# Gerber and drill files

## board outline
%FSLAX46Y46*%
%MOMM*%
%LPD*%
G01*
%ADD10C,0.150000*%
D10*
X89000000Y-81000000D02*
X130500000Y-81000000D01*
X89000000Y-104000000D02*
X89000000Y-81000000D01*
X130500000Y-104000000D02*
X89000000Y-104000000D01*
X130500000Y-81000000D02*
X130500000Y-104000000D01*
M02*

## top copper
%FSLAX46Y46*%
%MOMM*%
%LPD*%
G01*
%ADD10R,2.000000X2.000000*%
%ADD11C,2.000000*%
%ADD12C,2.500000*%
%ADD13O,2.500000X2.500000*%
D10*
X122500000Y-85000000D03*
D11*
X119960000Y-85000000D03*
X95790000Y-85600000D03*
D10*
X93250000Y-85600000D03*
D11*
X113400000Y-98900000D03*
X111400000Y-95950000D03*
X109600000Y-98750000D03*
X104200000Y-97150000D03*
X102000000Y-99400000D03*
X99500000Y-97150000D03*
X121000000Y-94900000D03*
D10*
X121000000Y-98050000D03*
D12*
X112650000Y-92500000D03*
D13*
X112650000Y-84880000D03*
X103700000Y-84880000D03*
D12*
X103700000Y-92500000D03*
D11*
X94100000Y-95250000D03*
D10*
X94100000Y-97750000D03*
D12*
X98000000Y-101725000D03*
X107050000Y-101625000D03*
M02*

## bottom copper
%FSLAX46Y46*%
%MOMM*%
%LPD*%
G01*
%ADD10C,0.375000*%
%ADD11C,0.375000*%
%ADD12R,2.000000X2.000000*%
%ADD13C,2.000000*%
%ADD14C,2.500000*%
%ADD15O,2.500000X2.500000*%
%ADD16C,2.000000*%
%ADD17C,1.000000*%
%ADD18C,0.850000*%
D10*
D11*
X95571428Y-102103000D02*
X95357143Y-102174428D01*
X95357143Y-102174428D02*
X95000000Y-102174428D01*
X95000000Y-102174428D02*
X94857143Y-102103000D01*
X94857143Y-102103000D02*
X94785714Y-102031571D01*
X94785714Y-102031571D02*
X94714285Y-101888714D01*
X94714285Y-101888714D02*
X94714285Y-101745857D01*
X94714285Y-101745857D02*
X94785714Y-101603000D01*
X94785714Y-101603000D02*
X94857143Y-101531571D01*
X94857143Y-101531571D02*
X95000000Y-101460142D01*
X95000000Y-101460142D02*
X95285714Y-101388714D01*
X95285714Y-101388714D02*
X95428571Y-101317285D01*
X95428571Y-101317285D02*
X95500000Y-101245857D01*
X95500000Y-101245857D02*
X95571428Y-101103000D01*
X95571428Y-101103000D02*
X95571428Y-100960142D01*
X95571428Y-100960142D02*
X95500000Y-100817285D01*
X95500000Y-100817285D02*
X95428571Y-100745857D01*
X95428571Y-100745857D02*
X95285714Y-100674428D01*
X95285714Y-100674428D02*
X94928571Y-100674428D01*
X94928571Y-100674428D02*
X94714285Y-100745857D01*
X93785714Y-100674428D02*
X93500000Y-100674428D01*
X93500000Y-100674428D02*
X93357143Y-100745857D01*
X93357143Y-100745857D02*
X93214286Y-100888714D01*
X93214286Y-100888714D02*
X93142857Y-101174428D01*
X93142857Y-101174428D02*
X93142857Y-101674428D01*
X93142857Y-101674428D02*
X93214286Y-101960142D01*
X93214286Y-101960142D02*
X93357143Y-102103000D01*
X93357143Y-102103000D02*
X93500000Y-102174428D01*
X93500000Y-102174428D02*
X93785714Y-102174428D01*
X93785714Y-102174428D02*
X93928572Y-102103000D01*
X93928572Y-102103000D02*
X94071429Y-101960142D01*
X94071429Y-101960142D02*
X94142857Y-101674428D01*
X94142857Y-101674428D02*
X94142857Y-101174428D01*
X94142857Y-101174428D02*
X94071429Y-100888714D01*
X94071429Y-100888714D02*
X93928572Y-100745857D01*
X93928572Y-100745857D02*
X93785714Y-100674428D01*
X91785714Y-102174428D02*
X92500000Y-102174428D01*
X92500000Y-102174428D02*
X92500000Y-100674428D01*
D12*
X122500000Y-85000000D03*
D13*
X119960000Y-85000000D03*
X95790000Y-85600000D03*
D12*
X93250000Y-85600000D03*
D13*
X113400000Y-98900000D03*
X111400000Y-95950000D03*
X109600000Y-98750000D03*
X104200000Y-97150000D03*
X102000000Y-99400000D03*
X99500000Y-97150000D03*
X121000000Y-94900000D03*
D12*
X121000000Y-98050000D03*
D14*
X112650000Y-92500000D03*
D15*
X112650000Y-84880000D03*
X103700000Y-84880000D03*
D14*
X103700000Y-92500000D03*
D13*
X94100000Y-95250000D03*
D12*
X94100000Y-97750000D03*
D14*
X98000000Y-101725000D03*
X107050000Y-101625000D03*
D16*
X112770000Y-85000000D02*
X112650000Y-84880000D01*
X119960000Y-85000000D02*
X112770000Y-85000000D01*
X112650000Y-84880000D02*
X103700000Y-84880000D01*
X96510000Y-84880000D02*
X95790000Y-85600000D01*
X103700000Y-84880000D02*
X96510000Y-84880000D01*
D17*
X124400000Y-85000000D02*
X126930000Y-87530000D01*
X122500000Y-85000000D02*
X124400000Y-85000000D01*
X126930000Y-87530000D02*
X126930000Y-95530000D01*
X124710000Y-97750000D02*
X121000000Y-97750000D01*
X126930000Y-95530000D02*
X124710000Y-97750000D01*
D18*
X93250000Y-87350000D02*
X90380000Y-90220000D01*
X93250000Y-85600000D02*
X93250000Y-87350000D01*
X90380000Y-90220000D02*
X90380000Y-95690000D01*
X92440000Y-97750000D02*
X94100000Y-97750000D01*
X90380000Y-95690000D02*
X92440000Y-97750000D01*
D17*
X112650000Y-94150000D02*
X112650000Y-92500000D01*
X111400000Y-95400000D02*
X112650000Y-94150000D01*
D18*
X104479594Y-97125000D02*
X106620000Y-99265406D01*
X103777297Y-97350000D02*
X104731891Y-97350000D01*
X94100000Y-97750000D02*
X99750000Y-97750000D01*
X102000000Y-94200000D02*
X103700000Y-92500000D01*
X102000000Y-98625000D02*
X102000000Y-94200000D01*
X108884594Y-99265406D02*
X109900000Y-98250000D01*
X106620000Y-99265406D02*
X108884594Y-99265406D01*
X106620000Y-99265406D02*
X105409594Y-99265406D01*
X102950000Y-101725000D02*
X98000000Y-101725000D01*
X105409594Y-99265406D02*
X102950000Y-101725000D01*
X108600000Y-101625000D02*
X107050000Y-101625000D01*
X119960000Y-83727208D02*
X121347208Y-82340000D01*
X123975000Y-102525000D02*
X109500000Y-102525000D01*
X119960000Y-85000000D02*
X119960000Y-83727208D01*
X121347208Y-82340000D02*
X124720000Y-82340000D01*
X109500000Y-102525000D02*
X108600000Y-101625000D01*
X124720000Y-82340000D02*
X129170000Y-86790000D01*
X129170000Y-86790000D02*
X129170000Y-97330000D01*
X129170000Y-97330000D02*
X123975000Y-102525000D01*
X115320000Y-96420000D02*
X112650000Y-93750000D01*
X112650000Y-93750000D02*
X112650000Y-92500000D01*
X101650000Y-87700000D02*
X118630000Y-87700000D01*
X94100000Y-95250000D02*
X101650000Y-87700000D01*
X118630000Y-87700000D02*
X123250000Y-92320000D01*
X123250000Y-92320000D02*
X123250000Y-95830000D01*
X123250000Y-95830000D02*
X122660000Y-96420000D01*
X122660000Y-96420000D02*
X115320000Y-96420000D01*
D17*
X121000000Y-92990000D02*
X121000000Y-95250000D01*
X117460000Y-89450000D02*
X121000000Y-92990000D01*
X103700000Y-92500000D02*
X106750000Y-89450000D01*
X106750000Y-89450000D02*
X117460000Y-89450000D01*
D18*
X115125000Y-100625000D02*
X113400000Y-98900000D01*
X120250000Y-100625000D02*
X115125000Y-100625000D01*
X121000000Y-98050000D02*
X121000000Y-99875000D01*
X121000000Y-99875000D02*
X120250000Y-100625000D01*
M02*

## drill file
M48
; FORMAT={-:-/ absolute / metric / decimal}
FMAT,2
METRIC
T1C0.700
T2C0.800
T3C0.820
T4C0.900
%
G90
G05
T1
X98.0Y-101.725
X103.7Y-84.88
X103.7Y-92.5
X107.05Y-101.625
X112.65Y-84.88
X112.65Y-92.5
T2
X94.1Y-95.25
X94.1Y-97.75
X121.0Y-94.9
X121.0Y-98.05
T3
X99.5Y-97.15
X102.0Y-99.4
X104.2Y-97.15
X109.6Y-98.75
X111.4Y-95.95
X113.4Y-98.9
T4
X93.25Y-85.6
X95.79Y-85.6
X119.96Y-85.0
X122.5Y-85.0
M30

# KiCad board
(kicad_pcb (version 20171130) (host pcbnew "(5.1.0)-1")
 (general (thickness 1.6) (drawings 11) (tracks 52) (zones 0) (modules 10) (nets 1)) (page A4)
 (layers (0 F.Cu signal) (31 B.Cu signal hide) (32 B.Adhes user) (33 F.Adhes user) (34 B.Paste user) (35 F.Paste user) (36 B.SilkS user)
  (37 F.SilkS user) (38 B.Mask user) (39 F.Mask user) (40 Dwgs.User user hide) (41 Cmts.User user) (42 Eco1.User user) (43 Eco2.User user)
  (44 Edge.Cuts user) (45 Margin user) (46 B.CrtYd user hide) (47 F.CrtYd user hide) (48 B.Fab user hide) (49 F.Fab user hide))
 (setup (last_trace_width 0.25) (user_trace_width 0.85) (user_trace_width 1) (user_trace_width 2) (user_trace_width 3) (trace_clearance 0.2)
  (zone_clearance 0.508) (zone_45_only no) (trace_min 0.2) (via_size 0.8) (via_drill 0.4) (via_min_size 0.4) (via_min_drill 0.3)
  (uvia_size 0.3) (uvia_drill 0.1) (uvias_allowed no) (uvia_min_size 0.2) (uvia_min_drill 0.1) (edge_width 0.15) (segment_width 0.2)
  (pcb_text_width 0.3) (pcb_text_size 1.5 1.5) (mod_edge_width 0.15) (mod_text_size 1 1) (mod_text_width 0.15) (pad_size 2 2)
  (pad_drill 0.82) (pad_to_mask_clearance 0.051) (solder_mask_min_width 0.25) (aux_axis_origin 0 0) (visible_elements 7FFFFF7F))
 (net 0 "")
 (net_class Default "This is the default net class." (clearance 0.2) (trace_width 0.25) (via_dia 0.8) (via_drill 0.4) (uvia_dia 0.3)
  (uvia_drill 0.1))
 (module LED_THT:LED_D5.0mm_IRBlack (layer F.Cu) (at 122.5 85 180)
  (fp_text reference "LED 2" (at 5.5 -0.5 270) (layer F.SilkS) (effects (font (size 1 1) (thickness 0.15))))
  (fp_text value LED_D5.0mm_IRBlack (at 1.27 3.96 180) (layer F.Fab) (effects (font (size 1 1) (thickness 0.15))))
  (pad 1 thru_hole rect (at 0 0 180) (size 2 2) (drill 0.9) (layers *.Cu *.Mask))
  (pad 2 thru_hole circle (at 2.54 0 180) (size 2 2) (drill 0.9) (layers *.Cu *.Mask)))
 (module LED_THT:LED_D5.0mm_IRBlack (layer F.Cu) (at 93.25 85.6)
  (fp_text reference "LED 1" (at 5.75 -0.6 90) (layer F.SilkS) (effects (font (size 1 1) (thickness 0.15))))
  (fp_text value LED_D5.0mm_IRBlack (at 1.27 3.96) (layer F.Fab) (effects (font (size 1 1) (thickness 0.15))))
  (pad 2 thru_hole circle (at 2.54 0) (size 2 2) (drill 0.9) (layers *.Cu *.Mask))
  (pad 1 thru_hole rect (at 0 0) (size 2 2) (drill 0.9) (layers *.Cu *.Mask)))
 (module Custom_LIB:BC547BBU (layer F.Cu) (at 111.4 97.85)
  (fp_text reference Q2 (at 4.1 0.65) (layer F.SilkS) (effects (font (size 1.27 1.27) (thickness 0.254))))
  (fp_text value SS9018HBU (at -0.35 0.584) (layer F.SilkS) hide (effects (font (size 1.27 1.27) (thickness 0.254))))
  (pad 3 thru_hole circle (at 2 1.05) (size 2 2) (drill 0.82) (layers *.Cu *.Mask))
  (pad 2 thru_hole circle (at 0 -1.9) (size 2 2) (drill 0.82) (layers *.Cu *.Mask))
  (pad 1 thru_hole circle (at -1.8 0.9) (size 2 2) (drill 0.82) (layers *.Cu *.Mask)))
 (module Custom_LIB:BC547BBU (layer F.Cu) (at 102 97.5 180)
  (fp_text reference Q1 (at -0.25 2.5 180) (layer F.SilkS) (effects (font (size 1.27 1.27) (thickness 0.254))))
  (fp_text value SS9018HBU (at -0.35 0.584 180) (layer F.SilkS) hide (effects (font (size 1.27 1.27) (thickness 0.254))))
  (pad 1 thru_hole circle (at -2.2 0.35 180) (size 2 2) (drill 0.82) (layers *.Cu *.Mask))
  (pad 2 thru_hole circle (at 0 -1.9 180) (size 2 2) (drill 0.82) (layers *.Cu *.Mask))
  (pad 3 thru_hole circle (at 2.5 0.35 180) (size 2 2) (drill 0.82) (layers *.Cu *.Mask)))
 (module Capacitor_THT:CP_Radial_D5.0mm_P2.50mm (layer F.Cu) (at 121 97.75 90)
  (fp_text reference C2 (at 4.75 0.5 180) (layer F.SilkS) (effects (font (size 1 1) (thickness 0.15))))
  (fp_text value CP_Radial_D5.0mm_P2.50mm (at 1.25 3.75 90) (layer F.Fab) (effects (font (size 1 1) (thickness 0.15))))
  (pad 2 thru_hole circle (at 2.85 0 90) (size 2 2) (drill 0.8) (layers *.Cu *.Mask))
  (pad 1 thru_hole rect (at -0.3 0 90) (size 2 2) (drill 0.8) (layers *.Cu *.Mask)))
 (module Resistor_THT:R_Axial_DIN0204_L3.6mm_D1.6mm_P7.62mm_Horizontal (layer F.Cu) (at 112.65 92.5 90)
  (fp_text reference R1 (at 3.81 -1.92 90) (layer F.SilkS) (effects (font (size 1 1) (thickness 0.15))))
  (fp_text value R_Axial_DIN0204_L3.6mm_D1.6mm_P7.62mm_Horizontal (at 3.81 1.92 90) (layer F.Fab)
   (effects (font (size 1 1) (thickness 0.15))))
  (pad 1 thru_hole circle (at 0 0 90) (size 2.5 2.5) (drill 0.7) (layers *.Cu *.Mask))
  (pad 2 thru_hole oval (at 7.62 0 90) (size 2.5 2.5) (drill 0.7) (layers *.Cu *.Mask)))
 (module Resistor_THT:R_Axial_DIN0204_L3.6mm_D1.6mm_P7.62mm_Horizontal (layer F.Cu) (at 103.7 92.5 90)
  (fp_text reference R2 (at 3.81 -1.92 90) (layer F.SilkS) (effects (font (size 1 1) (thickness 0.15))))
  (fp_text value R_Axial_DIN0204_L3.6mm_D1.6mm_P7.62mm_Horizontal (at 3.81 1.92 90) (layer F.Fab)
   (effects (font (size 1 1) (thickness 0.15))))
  (pad 2 thru_hole oval (at 7.62 0 90) (size 2.5 2.5) (drill 0.7) (layers *.Cu *.Mask))
  (pad 1 thru_hole circle (at 0 0 90) (size 2.5 2.5) (drill 0.7) (layers *.Cu *.Mask)))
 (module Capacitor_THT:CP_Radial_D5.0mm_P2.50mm (layer F.Cu) (at 94.1 97.75 90)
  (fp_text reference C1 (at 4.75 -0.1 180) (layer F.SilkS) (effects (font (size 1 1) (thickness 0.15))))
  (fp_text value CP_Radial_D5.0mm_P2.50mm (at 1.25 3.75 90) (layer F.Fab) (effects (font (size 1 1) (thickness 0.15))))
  (pad 2 thru_hole circle (at 2.5 0 90) (size 2 2) (drill 0.8) (layers *.Cu *.Mask))
  (pad 1 thru_hole rect (at 0 0 90) (size 2 2) (drill 0.8) (layers *.Cu *.Mask)))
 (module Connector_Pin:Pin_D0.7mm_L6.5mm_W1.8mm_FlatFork (layer F.Cu) (at 98 101.725)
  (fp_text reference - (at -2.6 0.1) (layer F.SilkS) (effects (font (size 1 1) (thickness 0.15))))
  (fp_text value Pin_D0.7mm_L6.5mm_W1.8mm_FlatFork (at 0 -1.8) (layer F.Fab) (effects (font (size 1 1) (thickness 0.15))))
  (pad 1 thru_hole circle (at 0 0) (size 2.5 2.5) (drill 0.7) (layers *.Cu *.Mask)))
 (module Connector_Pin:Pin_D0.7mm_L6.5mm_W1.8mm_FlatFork (layer F.Cu) (at 107.05 101.625)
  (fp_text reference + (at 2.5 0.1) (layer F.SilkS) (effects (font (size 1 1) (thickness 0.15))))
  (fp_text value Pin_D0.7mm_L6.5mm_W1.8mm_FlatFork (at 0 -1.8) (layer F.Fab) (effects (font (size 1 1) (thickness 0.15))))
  (pad 1 thru_hole circle (at 0 0) (size 2.5 2.5) (drill 0.7) (layers *.Cu *.Mask)))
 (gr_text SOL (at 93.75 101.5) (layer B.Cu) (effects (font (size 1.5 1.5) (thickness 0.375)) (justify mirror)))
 (gr_line (start 89 81) (end 130.5 81) (layer Edge.Cuts) (width 0.15))
 (gr_line (start 89 104) (end 89 81) (layer Edge.Cuts) (width 0.15))
 (gr_line (start 130.5 104) (end 89 104) (layer Edge.Cuts) (width 0.15))
 (gr_line (start 130.5 81) (end 130.5 104) (layer Edge.Cuts) (width 0.15))
 (segment (start 112.77 85) (end 112.65 84.88) (width 2) (layer B.Cu) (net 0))
 (segment (start 119.96 85) (end 112.77 85) (width 2) (layer B.Cu) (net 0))
 (segment (start 112.65 84.88) (end 103.7 84.88) (width 2) (layer B.Cu) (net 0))
 (segment (start 96.51 84.88) (end 95.79 85.6) (width 2) (layer B.Cu) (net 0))
 (segment (start 103.7 84.88) (end 96.51 84.88) (width 2) (layer B.Cu) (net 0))
 (segment (start 124.4 85) (end 126.93 87.53) (width 1) (layer B.Cu) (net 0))
 (segment (start 122.5 85) (end 124.4 85) (width 1) (layer B.Cu) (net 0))
 (segment (start 126.93 87.53) (end 126.93 95.53) (width 1) (layer B.Cu) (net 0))
 (segment (start 124.71 97.75) (end 121 97.75) (width 1) (layer B.Cu) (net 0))
 (segment (start 126.93 95.53) (end 124.71 97.75) (width 1) (layer B.Cu) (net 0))
 (segment (start 93.25 87.35) (end 90.38 90.22) (width 0.85) (layer B.Cu) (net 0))
 (segment (start 93.25 85.6) (end 93.25 87.35) (width 0.85) (layer B.Cu) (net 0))
 (segment (start 90.38 90.22) (end 90.38 95.69) (width 0.85) (layer B.Cu) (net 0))
 (segment (start 92.44 97.75) (end 94.1 97.75) (width 0.85) (layer B.Cu) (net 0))
 (segment (start 90.38 95.69) (end 92.44 97.75) (width 0.85) (layer B.Cu) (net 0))
 (segment (start 112.65 94.15) (end 112.65 92.5) (width 1) (layer B.Cu) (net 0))
 (segment (start 111.4 95.4) (end 112.65 94.15) (width 1) (layer B.Cu) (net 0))
 (segment (start 104.479594 97.125) (end 106.62 99.265406) (width 0.85) (layer B.Cu) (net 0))
 (segment (start 103.777297 97.35) (end 104.731891 97.35) (width 0.85) (layer B.Cu) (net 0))
 (segment (start 94.1 97.75) (end 99.75 97.75) (width 0.85) (layer B.Cu) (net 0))
 (segment (start 102 94.2) (end 103.7 92.5) (width 0.85) (layer B.Cu) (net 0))
 (segment (start 102 98.625) (end 102 94.2) (width 0.85) (layer B.Cu) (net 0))
 (segment (start 108.884594 99.265406) (end 109.9 98.25) (width 0.85) (layer B.Cu) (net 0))
 (segment (start 106.62 99.265406) (end 108.884594 99.265406) (width 0.85) (layer B.Cu) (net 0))
 (segment (start 106.62 99.265406) (end 105.409594 99.265406) (width 0.85) (layer B.Cu) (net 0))
 (segment (start 102.95 101.725) (end 98 101.725) (width 0.85) (layer B.Cu) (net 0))
 (segment (start 105.409594 99.265406) (end 102.95 101.725) (width 0.85) (layer B.Cu) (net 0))
 (segment (start 108.6 101.625) (end 107.05 101.625) (width 0.85) (layer B.Cu) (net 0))
 (segment (start 119.96 83.727208) (end 121.347208 82.34) (width 0.85) (layer B.Cu) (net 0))
 (segment (start 123.975 102.525) (end 109.5 102.525) (width 0.85) (layer B.Cu) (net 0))
 (segment (start 119.96 85) (end 119.96 83.727208) (width 0.85) (layer B.Cu) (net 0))
 (segment (start 121.347208 82.34) (end 124.72 82.34) (width 0.85) (layer B.Cu) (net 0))
 (segment (start 109.5 102.525) (end 108.6 101.625) (width 0.85) (layer B.Cu) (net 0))
 (segment (start 124.72 82.34) (end 129.17 86.79) (width 0.85) (layer B.Cu) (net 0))
 (segment (start 129.17 86.79) (end 129.17 97.33) (width 0.85) (layer B.Cu) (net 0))
 (segment (start 129.17 97.33) (end 123.975 102.525) (width 0.85) (layer B.Cu) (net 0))
 (segment (start 115.32 96.42) (end 112.65 93.75) (width 0.85) (layer B.Cu) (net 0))
 (segment (start 112.65 93.75) (end 112.65 92.5) (width 0.85) (layer B.Cu) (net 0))
 (segment (start 101.65 87.7) (end 118.63 87.7) (width 0.85) (layer B.Cu) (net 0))
 (segment (start 94.1 95.25) (end 101.65 87.7) (width 0.85) (layer B.Cu) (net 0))
 (segment (start 118.63 87.7) (end 123.25 92.32) (width 0.85) (layer B.Cu) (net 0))
 (segment (start 123.25 92.32) (end 123.25 95.83) (width 0.85) (layer B.Cu) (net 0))
 (segment (start 123.25 95.83) (end 122.66 96.42) (width 0.85) (layer B.Cu) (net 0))
 (segment (start 122.66 96.42) (end 115.32 96.42) (width 0.85) (layer B.Cu) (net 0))
 (segment (start 121 92.99) (end 121 95.25) (width 1) (layer B.Cu) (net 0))
 (segment (start 117.46 89.45) (end 121 92.99) (width 1) (layer B.Cu) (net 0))
 (segment (start 103.7 92.5) (end 106.75 89.45) (width 1) (layer B.Cu) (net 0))
 (segment (start 106.75 89.45) (end 117.46 89.45) (width 1) (layer B.Cu) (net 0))
 (segment (start 115.125 100.625) (end 113.4 98.9) (width 0.85) (layer B.Cu) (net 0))
 (segment (start 120.25 100.625) (end 115.125 100.625) (width 0.85) (layer B.Cu) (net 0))
 (segment (start 121 98.05) (end 121 99.875) (width 0.85) (layer B.Cu) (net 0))
 (segment (start 121 99.875) (end 120.25 100.625) (width 0.85) (layer B.Cu) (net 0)))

